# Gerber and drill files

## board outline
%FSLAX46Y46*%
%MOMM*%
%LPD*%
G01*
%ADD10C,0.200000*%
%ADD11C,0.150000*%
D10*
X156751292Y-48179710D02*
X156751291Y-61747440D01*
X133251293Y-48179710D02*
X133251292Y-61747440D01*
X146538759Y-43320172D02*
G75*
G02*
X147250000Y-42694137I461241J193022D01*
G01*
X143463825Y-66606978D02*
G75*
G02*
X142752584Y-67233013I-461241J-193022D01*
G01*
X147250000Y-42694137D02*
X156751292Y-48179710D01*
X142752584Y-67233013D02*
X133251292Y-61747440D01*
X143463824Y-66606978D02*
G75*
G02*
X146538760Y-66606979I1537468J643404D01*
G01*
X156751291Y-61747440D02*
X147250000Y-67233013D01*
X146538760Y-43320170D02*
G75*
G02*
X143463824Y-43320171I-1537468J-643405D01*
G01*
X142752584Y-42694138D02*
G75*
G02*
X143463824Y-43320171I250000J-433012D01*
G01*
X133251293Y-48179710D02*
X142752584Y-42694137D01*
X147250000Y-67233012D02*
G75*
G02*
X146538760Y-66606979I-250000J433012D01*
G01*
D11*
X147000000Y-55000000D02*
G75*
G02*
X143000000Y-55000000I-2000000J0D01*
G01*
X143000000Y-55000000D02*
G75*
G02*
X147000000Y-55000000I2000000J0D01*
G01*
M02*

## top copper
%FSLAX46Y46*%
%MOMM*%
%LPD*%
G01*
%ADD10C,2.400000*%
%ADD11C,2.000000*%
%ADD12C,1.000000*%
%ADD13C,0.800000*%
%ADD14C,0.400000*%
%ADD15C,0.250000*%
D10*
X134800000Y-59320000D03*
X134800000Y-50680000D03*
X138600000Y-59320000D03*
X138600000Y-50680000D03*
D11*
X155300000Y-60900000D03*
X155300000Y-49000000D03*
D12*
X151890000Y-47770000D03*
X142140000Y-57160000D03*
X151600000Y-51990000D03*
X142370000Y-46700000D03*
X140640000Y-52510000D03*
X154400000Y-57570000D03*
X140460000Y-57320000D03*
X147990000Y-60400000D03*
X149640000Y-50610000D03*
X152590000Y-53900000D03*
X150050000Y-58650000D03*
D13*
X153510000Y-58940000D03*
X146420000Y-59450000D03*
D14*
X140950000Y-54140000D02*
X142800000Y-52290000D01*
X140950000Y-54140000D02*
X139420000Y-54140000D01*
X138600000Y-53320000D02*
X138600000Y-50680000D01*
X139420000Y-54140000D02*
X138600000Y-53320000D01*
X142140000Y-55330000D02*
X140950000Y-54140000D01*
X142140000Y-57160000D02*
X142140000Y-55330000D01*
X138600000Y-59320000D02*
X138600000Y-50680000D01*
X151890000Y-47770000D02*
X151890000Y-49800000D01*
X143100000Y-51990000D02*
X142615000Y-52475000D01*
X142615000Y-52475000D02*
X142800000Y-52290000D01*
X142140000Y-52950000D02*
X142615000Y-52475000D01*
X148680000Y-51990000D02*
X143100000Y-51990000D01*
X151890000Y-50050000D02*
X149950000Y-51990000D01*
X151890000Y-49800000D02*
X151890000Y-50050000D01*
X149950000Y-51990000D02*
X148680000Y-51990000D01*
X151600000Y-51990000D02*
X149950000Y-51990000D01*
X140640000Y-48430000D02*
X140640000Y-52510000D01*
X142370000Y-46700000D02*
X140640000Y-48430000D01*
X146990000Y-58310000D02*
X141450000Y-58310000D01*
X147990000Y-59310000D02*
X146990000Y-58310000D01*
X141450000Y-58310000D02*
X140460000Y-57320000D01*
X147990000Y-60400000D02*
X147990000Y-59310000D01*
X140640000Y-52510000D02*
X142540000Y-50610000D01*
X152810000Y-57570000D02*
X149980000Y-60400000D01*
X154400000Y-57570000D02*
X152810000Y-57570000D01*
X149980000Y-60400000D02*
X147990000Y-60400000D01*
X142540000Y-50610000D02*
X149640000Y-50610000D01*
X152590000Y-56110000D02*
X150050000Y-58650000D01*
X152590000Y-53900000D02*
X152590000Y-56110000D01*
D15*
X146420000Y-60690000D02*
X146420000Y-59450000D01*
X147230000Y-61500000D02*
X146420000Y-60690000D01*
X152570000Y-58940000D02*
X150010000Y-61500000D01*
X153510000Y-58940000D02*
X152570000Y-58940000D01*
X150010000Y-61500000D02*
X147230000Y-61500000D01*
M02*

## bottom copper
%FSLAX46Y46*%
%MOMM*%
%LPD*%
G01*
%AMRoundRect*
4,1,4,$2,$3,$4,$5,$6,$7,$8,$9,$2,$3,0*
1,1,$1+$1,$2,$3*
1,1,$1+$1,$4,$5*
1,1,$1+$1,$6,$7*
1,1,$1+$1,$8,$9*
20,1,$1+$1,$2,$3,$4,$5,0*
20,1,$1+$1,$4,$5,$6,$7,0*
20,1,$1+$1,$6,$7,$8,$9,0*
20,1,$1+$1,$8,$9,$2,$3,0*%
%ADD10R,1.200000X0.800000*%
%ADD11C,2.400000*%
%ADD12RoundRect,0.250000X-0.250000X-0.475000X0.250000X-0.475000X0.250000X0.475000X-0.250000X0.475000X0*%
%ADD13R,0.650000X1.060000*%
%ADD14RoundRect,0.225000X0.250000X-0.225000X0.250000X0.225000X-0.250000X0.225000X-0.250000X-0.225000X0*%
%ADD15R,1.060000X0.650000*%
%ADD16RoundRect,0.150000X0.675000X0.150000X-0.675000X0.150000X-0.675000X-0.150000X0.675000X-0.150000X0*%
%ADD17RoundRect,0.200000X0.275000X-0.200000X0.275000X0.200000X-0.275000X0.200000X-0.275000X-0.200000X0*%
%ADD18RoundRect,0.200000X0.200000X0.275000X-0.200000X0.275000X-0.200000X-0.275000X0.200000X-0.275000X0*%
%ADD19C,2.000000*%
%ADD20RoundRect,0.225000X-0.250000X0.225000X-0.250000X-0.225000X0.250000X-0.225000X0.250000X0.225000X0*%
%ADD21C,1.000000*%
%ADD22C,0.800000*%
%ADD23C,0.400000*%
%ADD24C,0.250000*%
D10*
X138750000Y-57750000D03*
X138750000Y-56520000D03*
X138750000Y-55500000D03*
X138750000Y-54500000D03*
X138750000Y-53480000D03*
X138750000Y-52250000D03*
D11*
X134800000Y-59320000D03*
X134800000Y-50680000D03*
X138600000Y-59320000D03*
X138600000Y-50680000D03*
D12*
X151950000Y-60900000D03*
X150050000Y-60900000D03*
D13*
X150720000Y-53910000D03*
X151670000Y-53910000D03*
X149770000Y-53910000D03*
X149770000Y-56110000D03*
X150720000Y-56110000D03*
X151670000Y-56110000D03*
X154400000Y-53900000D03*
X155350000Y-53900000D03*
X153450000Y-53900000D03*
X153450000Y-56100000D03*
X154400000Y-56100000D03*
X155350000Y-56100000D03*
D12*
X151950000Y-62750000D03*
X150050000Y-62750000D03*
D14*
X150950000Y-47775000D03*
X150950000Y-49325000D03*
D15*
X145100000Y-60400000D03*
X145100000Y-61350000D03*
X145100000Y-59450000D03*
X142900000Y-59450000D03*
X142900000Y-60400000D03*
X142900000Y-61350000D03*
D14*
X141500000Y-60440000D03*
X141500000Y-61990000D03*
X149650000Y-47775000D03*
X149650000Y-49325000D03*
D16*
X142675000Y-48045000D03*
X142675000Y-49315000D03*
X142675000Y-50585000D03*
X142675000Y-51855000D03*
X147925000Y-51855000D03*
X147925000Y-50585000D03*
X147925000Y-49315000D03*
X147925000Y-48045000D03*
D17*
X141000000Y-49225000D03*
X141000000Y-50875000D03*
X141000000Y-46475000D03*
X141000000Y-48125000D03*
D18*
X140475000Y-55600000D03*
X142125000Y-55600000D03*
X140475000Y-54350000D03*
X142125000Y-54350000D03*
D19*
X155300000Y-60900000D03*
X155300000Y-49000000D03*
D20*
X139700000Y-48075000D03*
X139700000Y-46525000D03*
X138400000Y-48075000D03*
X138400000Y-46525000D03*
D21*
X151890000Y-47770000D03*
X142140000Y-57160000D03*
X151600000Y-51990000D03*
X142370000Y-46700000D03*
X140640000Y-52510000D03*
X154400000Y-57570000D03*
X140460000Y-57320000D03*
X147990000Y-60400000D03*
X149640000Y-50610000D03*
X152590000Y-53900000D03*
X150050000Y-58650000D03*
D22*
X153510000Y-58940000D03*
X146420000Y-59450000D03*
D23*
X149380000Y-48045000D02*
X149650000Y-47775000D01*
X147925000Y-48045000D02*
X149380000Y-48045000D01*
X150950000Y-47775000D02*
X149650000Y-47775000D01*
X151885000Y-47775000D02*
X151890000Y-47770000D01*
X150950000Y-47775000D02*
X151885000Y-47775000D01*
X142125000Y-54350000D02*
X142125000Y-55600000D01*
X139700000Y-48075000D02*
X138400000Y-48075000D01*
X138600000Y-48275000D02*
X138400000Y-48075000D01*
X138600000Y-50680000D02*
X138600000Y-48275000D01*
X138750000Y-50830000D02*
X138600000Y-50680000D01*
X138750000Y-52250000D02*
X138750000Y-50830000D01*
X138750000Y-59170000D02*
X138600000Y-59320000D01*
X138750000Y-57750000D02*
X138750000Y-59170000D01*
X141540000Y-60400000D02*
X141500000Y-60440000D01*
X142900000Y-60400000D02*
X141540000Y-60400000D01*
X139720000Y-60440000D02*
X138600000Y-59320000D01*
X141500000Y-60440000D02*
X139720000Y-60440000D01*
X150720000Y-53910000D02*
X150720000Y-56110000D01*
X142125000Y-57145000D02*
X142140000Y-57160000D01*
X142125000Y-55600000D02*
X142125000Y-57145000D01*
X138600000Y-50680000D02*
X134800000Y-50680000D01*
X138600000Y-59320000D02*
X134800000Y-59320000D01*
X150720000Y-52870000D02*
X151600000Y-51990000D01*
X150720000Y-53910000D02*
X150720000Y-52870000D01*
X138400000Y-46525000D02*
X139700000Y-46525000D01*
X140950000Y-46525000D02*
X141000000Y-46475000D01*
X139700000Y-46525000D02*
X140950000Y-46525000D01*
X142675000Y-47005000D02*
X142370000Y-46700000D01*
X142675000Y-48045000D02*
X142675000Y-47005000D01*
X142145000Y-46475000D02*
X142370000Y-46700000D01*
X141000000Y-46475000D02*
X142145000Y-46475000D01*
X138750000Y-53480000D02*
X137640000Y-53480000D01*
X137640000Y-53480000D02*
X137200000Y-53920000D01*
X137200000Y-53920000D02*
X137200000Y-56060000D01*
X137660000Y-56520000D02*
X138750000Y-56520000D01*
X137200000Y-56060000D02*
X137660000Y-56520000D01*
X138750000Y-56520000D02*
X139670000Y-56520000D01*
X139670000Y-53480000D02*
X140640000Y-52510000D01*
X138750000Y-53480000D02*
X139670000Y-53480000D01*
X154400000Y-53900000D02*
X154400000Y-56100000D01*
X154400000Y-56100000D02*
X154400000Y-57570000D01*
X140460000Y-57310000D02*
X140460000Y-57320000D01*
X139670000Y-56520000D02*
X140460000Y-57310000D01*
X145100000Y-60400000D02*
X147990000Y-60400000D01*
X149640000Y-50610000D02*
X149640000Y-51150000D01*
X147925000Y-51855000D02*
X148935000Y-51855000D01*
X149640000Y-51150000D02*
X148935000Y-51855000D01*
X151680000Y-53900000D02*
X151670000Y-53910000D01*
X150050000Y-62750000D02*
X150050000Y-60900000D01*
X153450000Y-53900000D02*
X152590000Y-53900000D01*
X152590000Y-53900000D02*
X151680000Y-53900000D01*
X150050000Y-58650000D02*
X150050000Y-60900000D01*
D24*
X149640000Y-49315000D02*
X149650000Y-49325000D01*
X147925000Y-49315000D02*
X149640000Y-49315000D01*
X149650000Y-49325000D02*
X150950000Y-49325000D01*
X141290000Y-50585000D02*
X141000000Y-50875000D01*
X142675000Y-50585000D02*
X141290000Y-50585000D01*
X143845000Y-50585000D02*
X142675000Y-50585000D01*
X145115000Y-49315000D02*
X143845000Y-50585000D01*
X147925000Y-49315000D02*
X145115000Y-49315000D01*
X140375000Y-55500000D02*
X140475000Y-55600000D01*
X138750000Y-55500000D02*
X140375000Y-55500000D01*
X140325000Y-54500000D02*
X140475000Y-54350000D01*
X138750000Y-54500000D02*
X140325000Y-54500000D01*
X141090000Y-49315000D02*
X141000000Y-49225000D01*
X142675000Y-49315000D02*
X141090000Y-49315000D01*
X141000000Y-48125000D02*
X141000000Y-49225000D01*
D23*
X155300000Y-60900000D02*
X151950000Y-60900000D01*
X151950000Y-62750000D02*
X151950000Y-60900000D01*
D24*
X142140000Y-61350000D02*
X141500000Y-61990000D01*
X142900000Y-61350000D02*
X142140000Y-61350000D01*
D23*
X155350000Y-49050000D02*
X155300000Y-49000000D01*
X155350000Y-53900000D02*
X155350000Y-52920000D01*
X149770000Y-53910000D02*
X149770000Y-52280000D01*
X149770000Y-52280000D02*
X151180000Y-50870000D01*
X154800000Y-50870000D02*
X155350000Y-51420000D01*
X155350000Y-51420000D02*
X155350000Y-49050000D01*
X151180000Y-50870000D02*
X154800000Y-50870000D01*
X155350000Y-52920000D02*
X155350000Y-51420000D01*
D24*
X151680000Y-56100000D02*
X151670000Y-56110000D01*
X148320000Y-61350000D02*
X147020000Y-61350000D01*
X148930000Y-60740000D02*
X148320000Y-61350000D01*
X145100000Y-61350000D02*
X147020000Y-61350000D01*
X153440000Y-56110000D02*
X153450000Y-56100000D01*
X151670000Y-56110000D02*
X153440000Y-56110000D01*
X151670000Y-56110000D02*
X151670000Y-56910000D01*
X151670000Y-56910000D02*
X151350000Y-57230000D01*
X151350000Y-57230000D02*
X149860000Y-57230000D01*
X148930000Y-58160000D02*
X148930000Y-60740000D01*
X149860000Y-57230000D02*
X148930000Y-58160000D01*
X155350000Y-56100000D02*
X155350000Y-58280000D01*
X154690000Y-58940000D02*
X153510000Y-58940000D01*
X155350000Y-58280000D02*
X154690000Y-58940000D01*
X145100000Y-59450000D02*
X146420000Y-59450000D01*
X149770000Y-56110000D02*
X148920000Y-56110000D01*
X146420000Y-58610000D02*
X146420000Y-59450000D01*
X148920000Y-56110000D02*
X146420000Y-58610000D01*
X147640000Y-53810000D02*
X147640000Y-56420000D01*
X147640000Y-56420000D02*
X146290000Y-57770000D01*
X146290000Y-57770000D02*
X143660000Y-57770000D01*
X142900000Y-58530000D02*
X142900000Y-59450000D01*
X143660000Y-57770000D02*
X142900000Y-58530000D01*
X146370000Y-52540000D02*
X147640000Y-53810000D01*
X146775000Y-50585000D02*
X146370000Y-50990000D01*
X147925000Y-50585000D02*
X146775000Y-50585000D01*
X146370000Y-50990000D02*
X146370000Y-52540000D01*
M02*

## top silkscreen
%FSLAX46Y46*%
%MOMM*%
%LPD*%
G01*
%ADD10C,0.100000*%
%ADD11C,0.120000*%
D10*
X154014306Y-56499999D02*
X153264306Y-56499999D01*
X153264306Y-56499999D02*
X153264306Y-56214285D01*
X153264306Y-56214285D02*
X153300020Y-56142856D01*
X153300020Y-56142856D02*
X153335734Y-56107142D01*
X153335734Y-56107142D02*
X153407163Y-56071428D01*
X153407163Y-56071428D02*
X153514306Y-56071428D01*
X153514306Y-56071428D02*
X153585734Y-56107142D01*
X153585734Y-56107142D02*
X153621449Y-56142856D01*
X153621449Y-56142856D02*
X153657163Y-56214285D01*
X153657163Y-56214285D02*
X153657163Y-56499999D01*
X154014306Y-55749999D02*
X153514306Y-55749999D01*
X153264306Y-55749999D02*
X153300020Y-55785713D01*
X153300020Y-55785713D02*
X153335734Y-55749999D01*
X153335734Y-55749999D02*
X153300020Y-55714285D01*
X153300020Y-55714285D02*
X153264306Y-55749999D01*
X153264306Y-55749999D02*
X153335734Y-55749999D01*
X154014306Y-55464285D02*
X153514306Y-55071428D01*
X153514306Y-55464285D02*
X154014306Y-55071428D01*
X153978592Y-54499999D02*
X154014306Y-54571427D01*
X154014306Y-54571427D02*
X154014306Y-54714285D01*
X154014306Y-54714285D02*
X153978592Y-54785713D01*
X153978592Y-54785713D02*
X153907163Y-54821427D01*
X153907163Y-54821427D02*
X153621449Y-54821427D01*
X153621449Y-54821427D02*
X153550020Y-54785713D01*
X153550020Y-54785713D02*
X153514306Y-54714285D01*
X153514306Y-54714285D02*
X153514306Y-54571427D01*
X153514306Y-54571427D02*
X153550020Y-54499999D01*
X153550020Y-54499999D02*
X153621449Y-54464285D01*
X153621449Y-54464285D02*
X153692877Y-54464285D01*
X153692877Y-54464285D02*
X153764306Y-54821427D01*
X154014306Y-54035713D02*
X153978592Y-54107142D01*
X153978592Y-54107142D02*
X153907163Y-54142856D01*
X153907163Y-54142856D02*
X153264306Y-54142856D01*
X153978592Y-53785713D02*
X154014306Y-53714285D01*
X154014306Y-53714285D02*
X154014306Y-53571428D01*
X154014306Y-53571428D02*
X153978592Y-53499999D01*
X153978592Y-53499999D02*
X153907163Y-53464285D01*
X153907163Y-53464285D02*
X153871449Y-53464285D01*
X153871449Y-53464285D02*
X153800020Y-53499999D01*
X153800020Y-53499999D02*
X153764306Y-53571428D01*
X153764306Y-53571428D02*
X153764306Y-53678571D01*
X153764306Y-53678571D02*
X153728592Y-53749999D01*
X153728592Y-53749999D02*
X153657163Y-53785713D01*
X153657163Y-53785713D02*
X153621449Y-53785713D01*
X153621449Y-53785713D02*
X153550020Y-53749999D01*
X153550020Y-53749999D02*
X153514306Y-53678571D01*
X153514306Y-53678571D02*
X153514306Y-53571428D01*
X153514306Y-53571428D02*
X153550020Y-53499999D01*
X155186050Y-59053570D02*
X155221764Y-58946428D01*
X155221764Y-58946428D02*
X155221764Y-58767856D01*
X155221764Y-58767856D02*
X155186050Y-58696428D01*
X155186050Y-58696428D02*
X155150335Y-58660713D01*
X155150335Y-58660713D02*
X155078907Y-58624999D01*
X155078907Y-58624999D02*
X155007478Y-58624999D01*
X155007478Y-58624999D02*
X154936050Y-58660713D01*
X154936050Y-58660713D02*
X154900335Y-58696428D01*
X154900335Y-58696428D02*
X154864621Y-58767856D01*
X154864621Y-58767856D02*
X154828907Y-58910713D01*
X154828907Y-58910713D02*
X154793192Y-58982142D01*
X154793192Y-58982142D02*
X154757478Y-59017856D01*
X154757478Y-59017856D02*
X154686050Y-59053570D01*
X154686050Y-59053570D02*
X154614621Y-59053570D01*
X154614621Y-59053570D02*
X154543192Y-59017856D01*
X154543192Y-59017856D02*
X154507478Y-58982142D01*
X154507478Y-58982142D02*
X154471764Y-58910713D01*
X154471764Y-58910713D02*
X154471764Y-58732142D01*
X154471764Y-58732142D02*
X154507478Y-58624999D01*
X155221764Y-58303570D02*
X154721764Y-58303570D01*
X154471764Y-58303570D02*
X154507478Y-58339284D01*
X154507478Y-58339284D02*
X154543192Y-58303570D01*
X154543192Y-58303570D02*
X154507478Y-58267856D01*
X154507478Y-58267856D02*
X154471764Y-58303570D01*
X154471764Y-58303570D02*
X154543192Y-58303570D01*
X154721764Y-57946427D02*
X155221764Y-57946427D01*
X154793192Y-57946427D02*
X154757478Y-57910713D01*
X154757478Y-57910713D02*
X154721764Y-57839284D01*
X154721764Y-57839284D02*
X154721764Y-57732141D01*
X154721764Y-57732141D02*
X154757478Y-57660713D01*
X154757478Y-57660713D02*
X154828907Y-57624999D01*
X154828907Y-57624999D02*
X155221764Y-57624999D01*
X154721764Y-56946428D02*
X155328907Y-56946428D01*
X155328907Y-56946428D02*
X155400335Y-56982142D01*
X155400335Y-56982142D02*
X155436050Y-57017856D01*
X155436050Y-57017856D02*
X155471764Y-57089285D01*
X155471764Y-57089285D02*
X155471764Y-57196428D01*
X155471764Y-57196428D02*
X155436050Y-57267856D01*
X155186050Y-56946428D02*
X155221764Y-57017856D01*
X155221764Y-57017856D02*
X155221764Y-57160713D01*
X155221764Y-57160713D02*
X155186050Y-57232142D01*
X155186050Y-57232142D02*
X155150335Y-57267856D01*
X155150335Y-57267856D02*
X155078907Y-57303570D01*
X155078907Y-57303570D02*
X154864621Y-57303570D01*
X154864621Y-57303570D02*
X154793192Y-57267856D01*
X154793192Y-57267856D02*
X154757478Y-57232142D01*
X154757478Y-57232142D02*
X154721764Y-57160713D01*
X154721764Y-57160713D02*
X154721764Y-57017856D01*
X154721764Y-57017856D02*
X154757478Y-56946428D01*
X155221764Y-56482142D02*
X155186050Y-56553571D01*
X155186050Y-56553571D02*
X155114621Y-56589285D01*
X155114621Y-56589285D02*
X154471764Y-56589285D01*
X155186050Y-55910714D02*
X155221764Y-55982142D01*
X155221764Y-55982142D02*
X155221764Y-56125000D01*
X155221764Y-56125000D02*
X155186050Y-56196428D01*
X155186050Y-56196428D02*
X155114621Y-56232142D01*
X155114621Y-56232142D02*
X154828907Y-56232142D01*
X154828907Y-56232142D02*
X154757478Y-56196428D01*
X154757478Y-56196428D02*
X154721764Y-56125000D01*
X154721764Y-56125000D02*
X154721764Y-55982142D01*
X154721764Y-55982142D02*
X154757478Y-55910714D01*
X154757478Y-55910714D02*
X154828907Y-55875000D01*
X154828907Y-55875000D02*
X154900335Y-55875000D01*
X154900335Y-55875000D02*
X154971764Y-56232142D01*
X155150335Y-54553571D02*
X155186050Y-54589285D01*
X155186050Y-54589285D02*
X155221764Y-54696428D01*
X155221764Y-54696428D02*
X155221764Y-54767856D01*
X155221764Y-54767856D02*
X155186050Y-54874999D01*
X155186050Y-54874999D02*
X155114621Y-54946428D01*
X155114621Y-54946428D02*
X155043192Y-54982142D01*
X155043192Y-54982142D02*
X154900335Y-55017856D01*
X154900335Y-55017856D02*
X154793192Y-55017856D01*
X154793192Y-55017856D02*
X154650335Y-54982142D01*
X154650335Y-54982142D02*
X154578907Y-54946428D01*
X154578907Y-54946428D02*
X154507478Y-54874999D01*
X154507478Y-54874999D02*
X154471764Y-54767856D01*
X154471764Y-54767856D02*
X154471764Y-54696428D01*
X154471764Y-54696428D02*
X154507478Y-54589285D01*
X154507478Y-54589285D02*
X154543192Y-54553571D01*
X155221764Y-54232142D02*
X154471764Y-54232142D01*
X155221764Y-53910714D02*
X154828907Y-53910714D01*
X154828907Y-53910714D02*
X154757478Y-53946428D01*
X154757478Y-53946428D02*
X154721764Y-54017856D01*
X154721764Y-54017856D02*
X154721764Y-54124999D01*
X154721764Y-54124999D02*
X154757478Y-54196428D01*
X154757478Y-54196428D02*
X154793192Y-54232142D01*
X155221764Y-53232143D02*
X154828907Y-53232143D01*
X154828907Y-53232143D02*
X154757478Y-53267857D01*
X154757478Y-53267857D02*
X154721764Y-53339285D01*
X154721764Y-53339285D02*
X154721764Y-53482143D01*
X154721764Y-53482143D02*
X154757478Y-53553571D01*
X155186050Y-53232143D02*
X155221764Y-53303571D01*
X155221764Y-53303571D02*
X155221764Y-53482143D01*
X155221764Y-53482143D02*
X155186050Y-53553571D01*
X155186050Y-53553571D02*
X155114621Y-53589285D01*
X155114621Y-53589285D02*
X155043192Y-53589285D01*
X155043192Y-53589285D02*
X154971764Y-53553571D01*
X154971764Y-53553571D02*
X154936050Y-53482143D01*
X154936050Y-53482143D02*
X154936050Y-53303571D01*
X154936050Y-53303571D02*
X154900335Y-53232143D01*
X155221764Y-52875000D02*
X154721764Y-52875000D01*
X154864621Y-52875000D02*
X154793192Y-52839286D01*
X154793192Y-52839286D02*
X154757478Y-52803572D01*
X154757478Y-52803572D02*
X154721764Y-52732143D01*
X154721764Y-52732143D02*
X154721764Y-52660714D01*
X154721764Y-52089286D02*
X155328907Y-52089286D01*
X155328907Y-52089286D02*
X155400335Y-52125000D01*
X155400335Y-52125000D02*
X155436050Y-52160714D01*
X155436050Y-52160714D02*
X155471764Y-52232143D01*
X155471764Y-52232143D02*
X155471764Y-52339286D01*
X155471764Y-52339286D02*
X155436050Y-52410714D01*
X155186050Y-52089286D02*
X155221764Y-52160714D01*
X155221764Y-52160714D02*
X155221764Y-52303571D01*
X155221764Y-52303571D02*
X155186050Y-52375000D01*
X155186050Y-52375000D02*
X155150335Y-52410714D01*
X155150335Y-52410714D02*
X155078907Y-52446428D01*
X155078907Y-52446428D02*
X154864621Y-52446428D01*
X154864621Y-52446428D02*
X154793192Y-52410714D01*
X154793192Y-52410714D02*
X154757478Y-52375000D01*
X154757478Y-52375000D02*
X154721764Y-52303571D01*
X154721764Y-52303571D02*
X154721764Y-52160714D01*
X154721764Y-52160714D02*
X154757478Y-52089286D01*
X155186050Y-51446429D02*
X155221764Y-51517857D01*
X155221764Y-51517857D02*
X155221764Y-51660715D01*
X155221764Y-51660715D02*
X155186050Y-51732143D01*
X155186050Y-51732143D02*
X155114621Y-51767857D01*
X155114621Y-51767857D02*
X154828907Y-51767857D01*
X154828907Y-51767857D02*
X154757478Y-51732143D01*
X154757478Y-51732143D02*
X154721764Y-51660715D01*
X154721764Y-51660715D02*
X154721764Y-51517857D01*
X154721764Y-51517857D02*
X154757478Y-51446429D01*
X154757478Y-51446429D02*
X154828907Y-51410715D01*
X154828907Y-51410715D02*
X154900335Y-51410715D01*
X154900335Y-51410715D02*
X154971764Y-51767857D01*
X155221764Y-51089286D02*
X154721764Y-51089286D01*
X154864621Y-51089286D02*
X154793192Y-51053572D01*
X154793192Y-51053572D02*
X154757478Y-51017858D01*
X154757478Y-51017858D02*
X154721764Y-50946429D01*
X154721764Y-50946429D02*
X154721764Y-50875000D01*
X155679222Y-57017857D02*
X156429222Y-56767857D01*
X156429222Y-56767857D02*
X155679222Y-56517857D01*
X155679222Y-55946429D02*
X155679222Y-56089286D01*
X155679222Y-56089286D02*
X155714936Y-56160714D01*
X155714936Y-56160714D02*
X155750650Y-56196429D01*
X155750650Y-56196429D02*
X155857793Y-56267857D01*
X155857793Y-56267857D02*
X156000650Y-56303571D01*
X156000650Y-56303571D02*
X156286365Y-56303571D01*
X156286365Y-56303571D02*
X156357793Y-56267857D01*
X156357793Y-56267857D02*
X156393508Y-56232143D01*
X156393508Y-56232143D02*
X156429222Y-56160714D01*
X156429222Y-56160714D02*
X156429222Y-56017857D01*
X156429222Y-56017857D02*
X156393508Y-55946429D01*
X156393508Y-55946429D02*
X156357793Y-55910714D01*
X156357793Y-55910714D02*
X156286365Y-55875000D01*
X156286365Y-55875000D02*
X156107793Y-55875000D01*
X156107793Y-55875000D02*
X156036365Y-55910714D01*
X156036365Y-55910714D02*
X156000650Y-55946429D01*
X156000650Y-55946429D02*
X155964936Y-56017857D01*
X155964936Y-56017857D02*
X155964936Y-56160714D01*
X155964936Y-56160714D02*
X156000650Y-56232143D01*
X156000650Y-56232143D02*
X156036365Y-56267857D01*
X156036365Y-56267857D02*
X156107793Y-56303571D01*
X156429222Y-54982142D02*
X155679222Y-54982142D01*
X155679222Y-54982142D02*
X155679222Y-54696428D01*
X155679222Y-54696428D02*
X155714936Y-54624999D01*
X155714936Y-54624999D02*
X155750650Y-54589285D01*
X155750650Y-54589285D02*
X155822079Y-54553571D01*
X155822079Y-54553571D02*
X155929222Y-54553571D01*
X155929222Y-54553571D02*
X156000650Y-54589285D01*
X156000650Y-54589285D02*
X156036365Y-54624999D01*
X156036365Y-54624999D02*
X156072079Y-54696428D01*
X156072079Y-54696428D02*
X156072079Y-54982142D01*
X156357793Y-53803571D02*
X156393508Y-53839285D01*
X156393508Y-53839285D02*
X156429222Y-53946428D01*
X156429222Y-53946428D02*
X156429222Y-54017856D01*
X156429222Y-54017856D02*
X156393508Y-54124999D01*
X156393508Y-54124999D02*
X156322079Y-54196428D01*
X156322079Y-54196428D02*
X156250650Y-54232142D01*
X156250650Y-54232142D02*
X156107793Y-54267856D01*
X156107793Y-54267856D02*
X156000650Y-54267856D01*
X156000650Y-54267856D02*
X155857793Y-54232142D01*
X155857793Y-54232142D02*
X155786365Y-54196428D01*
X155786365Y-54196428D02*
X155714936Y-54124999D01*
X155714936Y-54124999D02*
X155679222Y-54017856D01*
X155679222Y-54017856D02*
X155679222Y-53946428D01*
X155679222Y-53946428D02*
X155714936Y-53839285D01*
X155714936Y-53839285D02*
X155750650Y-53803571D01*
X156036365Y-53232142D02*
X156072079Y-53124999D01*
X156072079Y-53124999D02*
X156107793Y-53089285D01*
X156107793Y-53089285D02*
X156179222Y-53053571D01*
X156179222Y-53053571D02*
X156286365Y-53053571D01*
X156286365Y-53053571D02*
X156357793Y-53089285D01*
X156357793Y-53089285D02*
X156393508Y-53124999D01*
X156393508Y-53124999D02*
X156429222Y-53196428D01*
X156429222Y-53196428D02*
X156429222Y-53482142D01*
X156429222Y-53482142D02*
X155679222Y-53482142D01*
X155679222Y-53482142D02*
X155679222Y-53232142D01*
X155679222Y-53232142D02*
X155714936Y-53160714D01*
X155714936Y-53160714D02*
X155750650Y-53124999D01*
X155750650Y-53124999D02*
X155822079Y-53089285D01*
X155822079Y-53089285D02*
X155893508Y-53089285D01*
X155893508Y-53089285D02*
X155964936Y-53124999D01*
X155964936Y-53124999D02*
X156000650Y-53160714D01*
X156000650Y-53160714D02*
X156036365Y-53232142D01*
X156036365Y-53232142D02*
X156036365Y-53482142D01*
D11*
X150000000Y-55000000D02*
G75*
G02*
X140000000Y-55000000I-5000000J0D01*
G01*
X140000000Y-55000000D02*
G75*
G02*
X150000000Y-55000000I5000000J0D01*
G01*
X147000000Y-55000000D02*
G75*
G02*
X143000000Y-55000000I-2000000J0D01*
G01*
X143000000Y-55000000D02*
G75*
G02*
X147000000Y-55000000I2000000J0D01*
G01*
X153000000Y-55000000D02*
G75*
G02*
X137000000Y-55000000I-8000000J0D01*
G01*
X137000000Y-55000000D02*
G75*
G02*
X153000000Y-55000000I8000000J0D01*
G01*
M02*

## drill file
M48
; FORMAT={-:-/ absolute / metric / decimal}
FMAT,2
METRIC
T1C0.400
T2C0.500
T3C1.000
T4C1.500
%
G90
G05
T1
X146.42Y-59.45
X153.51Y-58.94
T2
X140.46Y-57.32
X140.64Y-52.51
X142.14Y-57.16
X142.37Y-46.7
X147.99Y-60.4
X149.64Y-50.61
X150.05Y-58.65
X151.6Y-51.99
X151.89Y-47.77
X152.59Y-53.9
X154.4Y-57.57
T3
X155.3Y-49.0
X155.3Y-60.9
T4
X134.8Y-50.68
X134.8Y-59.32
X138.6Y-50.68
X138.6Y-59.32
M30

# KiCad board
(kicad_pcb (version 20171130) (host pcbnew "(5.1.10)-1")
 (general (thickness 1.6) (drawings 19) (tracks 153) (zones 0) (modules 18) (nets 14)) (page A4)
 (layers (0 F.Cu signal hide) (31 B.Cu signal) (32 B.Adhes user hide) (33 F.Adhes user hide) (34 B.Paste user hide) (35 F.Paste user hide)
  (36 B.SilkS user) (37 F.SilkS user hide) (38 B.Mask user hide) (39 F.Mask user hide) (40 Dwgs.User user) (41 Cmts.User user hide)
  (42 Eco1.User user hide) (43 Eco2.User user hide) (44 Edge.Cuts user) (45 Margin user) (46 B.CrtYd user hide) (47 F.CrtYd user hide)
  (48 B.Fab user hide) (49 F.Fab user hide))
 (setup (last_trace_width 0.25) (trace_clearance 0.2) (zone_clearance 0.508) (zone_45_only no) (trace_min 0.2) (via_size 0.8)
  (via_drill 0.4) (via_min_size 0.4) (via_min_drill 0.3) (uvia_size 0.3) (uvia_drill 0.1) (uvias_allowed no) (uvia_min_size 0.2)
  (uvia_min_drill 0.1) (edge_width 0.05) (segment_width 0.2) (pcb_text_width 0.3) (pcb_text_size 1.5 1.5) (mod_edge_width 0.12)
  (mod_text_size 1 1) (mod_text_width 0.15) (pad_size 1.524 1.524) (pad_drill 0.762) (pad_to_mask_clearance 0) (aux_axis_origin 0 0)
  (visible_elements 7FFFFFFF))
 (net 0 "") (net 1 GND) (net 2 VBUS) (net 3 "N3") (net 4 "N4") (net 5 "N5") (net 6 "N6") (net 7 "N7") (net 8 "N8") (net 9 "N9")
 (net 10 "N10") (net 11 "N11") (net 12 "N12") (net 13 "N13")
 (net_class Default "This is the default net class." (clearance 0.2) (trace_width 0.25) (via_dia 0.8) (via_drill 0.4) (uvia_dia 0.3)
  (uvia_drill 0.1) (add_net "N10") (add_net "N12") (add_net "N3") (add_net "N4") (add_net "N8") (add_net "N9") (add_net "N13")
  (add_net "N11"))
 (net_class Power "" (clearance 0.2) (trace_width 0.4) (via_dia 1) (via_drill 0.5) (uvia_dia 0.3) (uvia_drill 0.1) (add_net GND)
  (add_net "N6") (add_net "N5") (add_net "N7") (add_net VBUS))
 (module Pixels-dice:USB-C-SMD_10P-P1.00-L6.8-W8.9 (layer B.Cu) (at 136.7 55)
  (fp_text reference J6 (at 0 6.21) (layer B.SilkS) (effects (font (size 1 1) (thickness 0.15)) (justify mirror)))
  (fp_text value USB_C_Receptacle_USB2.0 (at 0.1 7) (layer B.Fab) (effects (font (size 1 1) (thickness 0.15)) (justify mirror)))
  (pad B12 smd rect (at 2.05 2.75 90) (size 0.8 1.2) (layers B.Cu B.Paste B.Mask) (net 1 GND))
  (pad B9 smd rect (at 2.05 1.52 90) (size 0.8 1.2) (layers B.Cu B.Paste B.Mask) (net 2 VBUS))
  (pad A5 smd rect (at 2.05 0.5 90) (size 0.8 1.2) (layers B.Cu B.Paste B.Mask) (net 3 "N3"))
  (pad B5 smd rect (at 2.05 -0.5 90) (size 0.8 1.2) (layers B.Cu B.Paste B.Mask) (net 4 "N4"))
  (pad A9 smd rect (at 2.05 -1.52 90) (size 0.8 1.2) (layers B.Cu B.Paste B.Mask) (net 2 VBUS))
  (pad A12 smd rect (at 2.05 -2.75 90) (size 0.8 1.2) (layers B.Cu B.Paste B.Mask) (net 1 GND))
  (pad S1 thru_hole circle (at -1.9 4.32 90) (size 2.4 2.4) (drill 1.5) (layers *.Cu *.Mask) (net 1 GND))
  (pad S1 thru_hole circle (at -1.9 -4.32 90) (size 2.4 2.4) (drill 1.5) (layers *.Cu *.Mask) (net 1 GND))
  (pad S1 thru_hole circle (at 1.9 4.32 90) (size 2.4 2.4) (drill 1.5) (layers *.Cu *.Mask) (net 1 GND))
  (pad S1 thru_hole circle (at 1.9 -4.32 90) (size 2.4 2.4) (drill 1.5) (layers *.Cu *.Mask) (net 1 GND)))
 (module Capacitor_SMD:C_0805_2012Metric (layer B.Cu) (at 151 60.9)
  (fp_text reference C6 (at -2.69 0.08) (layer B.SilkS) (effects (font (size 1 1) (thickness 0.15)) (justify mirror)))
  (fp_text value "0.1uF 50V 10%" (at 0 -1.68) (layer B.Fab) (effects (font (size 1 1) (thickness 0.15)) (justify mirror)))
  (pad 2 smd roundrect (at 0.95 0) (size 1 1.45) (layers B.Cu B.Paste B.Mask) (roundrect_rratio 0.25) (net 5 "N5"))
  (pad 1 smd roundrect (at -0.95 0) (size 1 1.45) (layers B.Cu B.Paste B.Mask) (roundrect_rratio 0.25) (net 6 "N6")))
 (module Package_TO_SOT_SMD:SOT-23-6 (layer B.Cu) (at 150.72 55.01 90)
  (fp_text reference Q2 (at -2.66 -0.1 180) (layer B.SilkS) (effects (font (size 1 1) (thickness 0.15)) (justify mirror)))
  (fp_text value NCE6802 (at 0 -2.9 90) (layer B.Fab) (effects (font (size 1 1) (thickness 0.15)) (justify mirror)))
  (pad 5 smd rect (at 1.1 0 90) (size 1.06 0.65) (layers B.Cu B.Paste B.Mask) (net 1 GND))
  (pad 6 smd rect (at 1.1 0.95 90) (size 1.06 0.65) (layers B.Cu B.Paste B.Mask) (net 6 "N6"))
  (pad 4 smd rect (at 1.1 -0.95 90) (size 1.06 0.65) (layers B.Cu B.Paste B.Mask) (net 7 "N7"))
  (pad 3 smd rect (at -1.1 -0.95 90) (size 1.06 0.65) (layers B.Cu B.Paste B.Mask) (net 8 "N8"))
  (pad 2 smd rect (at -1.1 0 90) (size 1.06 0.65) (layers B.Cu B.Paste B.Mask) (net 1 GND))
  (pad 1 smd rect (at -1.1 0.95 90) (size 1.06 0.65) (layers B.Cu B.Paste B.Mask) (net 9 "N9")))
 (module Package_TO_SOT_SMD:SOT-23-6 (layer B.Cu) (at 154.4 55 90)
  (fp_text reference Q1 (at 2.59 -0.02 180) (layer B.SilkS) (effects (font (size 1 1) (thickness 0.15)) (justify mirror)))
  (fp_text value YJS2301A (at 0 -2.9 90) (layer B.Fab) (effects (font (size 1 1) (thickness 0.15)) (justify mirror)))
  (pad 5 smd rect (at 1.1 0 90) (size 1.06 0.65) (layers B.Cu B.Paste B.Mask) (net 2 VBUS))
  (pad 6 smd rect (at 1.1 0.95 90) (size 1.06 0.65) (layers B.Cu B.Paste B.Mask) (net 7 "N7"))
  (pad 4 smd rect (at 1.1 -0.95 90) (size 1.06 0.65) (layers B.Cu B.Paste B.Mask) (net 6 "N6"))
  (pad 3 smd rect (at -1.1 -0.95 90) (size 1.06 0.65) (layers B.Cu B.Paste B.Mask) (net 9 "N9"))
  (pad 2 smd rect (at -1.1 0 90) (size 1.06 0.65) (layers B.Cu B.Paste B.Mask) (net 2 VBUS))
  (pad 1 smd rect (at -1.1 0.95 90) (size 1.06 0.65) (layers B.Cu B.Paste B.Mask) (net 8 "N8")))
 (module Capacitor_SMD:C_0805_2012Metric (layer B.Cu) (at 151 62.75)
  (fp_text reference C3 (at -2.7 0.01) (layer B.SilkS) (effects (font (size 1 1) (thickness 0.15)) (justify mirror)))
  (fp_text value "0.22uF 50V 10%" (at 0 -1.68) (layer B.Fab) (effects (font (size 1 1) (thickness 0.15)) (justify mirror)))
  (pad 2 smd roundrect (at 0.95 0) (size 1 1.45) (layers B.Cu B.Paste B.Mask) (roundrect_rratio 0.25) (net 5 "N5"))
  (pad 1 smd roundrect (at -0.95 0) (size 1 1.45) (layers B.Cu B.Paste B.Mask) (roundrect_rratio 0.25) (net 6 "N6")))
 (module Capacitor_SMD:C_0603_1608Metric (layer B.Cu) (at 150.95 48.55 90)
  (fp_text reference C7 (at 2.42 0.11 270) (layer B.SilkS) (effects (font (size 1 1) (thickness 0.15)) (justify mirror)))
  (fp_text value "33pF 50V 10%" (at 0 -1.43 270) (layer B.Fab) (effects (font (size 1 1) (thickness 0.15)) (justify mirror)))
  (pad 2 smd roundrect (at 0.775 0 90) (size 0.9 0.95) (layers B.Cu B.Paste B.Mask) (roundrect_rratio 0.25) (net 1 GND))
  (pad 1 smd roundrect (at -0.775 0 90) (size 0.9 0.95) (layers B.Cu B.Paste B.Mask) (roundrect_rratio 0.25) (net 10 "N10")))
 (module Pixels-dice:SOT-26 (layer B.Cu) (at 144 60.4 180)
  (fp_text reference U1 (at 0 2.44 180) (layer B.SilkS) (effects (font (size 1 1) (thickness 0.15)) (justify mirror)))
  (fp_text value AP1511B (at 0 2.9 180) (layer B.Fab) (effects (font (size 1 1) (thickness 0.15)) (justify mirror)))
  (pad 5 smd rect (at -1.1 0) (size 1.06 0.65) (layers B.Cu B.Paste B.Mask) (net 2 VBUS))
  (pad 6 smd rect (at -1.1 -0.95) (size 1.06 0.65) (layers B.Cu B.Paste B.Mask) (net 9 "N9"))
  (pad 4 smd rect (at -1.1 0.95) (size 1.06 0.65) (layers B.Cu B.Paste B.Mask) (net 8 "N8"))
  (pad 3 smd rect (at 1.1 0.95) (size 1.06 0.65) (layers B.Cu B.Paste B.Mask) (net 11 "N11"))
  (pad 2 smd rect (at 1.1 0) (size 1.06 0.65) (layers B.Cu B.Paste B.Mask) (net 1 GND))
  (pad 1 smd rect (at 1.1 -0.95) (size 1.06 0.65) (layers B.Cu B.Paste B.Mask) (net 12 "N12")))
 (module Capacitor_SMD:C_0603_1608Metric (layer B.Cu) (at 141.5 61.215 90)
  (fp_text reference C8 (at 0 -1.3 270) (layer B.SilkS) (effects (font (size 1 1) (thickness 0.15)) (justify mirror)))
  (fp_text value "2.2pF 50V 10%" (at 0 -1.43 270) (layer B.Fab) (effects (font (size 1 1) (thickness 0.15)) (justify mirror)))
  (pad 2 smd roundrect (at 0.775 0 90) (size 0.9 0.95) (layers B.Cu B.Paste B.Mask) (roundrect_rratio 0.25) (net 1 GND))
  (pad 1 smd roundrect (at -0.775 0 90) (size 0.9 0.95) (layers B.Cu B.Paste B.Mask) (roundrect_rratio 0.25) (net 12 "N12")))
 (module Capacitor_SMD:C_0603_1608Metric (layer B.Cu) (at 149.65 48.55 90)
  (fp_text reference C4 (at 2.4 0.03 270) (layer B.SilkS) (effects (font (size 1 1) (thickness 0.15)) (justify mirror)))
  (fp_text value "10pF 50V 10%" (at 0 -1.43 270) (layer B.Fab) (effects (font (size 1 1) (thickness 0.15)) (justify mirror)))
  (pad 2 smd roundrect (at 0.775 0 90) (size 0.9 0.95) (layers B.Cu B.Paste B.Mask) (roundrect_rratio 0.25) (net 1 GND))
  (pad 1 smd roundrect (at -0.775 0 90) (size 0.9 0.95) (layers B.Cu B.Paste B.Mask) (roundrect_rratio 0.25) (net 10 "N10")))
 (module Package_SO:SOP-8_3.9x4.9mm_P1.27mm (layer B.Cu) (at 145.3 49.95 180)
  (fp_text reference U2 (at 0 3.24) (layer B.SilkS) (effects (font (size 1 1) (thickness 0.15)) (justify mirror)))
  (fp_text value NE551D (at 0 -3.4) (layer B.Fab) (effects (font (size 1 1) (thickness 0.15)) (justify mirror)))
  (pad 8 smd roundrect (at 2.625 1.905 180) (size 1.65 0.6) (layers B.Cu B.Paste B.Mask) (roundrect_rratio 0.25) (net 2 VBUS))
  (pad 7 smd roundrect (at 2.625 0.635 180) (size 1.65 0.6) (layers B.Cu B.Paste B.Mask) (roundrect_rratio 0.25) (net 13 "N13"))
  (pad 6 smd roundrect (at 2.625 -0.635 180) (size 1.65 0.6) (layers B.Cu B.Paste B.Mask) (roundrect_rratio 0.25) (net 10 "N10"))
  (pad 5 smd roundrect (at 2.625 -1.905 180) (size 1.65 0.6) (layers B.Cu B.Paste B.Mask) (roundrect_rratio 0.25))
  (pad 4 smd roundrect (at -2.625 -1.905 180) (size 1.65 0.6) (layers B.Cu B.Paste B.Mask) (roundrect_rratio 0.25) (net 2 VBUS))
  (pad 3 smd roundrect (at -2.625 -0.635 180) (size 1.65 0.6) (layers B.Cu B.Paste B.Mask) (roundrect_rratio 0.25) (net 11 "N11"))
  (pad 2 smd roundrect (at -2.625 0.635 180) (size 1.65 0.6) (layers B.Cu B.Paste B.Mask) (roundrect_rratio 0.25) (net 10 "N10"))
  (pad 1 smd roundrect (at -2.625 1.905 180) (size 1.65 0.6) (layers B.Cu B.Paste B.Mask) (roundrect_rratio 0.25) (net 1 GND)))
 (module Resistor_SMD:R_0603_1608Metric (layer B.Cu) (at 141 50.05 90)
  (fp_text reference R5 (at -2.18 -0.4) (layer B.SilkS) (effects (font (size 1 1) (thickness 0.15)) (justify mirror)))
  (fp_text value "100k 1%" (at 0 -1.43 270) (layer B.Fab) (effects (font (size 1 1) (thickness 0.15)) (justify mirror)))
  (pad 2 smd roundrect (at 0.825 0 90) (size 0.8 0.95) (layers B.Cu B.Paste B.Mask) (roundrect_rratio 0.25) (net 13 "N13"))
  (pad 1 smd roundrect (at -0.825 0 90) (size 0.8 0.95) (layers B.Cu B.Paste B.Mask) (roundrect_rratio 0.25) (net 10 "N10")))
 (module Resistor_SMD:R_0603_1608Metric (layer B.Cu) (at 141 47.3 90)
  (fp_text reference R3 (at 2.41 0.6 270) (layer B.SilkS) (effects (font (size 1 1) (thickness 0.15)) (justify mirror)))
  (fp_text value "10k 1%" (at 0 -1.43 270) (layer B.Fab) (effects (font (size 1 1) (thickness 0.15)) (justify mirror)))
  (pad 2 smd roundrect (at 0.825 0 90) (size 0.8 0.95) (layers B.Cu B.Paste B.Mask) (roundrect_rratio 0.25) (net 2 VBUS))
  (pad 1 smd roundrect (at -0.825 0 90) (size 0.8 0.95) (layers B.Cu B.Paste B.Mask) (roundrect_rratio 0.25) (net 13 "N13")))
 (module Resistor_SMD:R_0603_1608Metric (layer B.Cu) (at 141.3 55.6 180)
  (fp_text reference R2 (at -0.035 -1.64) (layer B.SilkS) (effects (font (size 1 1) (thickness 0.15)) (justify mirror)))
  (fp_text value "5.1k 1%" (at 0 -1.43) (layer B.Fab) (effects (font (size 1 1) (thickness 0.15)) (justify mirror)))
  (pad 2 smd roundrect (at 0.825 0 180) (size 0.8 0.95) (layers B.Cu B.Paste B.Mask) (roundrect_rratio 0.25) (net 3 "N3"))
  (pad 1 smd roundrect (at -0.825 0 180) (size 0.8 0.95) (layers B.Cu B.Paste B.Mask) (roundrect_rratio 0.25) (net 1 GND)))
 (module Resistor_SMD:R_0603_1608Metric (layer B.Cu) (at 141.3 54.35 180)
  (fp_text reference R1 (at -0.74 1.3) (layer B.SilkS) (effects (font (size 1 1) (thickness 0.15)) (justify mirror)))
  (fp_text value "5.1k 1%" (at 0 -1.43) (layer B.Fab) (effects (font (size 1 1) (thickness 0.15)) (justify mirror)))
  (pad 2 smd roundrect (at 0.825 0 180) (size 0.8 0.95) (layers B.Cu B.Paste B.Mask) (roundrect_rratio 0.25) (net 4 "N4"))
  (pad 1 smd roundrect (at -0.825 0 180) (size 0.8 0.95) (layers B.Cu B.Paste B.Mask) (roundrect_rratio 0.25) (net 1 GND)))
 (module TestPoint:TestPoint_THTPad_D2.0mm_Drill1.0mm (layer B.Cu) (at 155.3 60.9)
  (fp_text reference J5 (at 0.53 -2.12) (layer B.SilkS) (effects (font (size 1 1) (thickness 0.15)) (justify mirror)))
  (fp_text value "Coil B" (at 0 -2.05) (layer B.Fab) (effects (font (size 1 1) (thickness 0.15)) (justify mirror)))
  (pad 1 thru_hole circle (at 0 0) (size 2 2) (drill 1) (layers *.Cu *.Mask) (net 5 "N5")))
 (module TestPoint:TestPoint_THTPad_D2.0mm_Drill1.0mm (layer B.Cu) (at 155.3 49)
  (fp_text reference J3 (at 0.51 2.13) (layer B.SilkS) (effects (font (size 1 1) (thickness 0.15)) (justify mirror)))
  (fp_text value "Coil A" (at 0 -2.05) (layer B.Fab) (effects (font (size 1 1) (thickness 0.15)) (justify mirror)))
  (pad 1 thru_hole circle (at 0 0) (size 2 2) (drill 1) (layers *.Cu *.Mask) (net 7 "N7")))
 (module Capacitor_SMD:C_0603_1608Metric (layer B.Cu) (at 139.7 47.3 270)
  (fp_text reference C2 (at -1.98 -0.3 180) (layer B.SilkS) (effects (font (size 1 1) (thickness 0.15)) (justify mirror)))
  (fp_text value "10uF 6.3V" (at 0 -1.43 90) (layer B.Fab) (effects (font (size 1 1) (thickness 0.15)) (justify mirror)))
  (pad 2 smd roundrect (at 0.775 0 270) (size 0.9 0.95) (layers B.Cu B.Paste B.Mask) (roundrect_rratio 0.25) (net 1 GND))
  (pad 1 smd roundrect (at -0.775 0 270) (size 0.9 0.95) (layers B.Cu B.Paste B.Mask) (roundrect_rratio 0.25) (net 2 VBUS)))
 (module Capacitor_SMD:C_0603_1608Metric (layer B.Cu) (at 138.4 47.3 270)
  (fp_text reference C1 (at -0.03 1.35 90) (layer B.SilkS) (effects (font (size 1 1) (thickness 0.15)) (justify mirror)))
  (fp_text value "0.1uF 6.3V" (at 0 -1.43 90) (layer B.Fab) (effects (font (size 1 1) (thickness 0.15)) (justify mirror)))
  (pad 2 smd roundrect (at 0.775 0 270) (size 0.9 0.95) (layers B.Cu B.Paste B.Mask) (roundrect_rratio 0.25) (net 1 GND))
  (pad 1 smd roundrect (at -0.775 0 270) (size 0.9 0.95) (layers B.Cu B.Paste B.Mask) (roundrect_rratio 0.25) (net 2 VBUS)))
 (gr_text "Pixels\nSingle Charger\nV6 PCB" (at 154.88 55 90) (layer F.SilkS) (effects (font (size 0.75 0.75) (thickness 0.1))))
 (gr_line (start 156.751292 48.17971) (end 156.751291 61.74744) (layer Edge.Cuts) (width 0.2))
 (gr_line (start 133.251293 48.17971) (end 133.251292 61.74744) (layer Edge.Cuts) (width 0.2))
 (gr_circle (center 145 55) (end 150 55) (layer F.SilkS) (width 0.12))
 (gr_circle (center 145 55) (end 147 55) (layer F.SilkS) (width 0.12))
 (gr_circle (center 145 55) (end 153 55) (layer F.SilkS) (width 0.12))
 (gr_arc (start 147 43.12715) (end 147.25 42.694137) (angle -142.7084941) (layer Edge.Cuts) (width 0.2))
 (gr_arc (start 143.002584 66.8) (end 142.752584 67.233013) (angle -142.7084941) (layer Edge.Cuts) (width 0.2))
 (gr_line (start 147.25 42.694137) (end 156.751292 48.17971) (layer Edge.Cuts) (width 0.2))
 (gr_line (start 142.752584 67.233013) (end 133.251292 61.74744) (layer Edge.Cuts) (width 0.2))
 (gr_arc (start 145.001292 65.963574) (end 146.53876 66.606979) (angle -225.4169678) (layer Edge.Cuts) (width 0.2))
 (gr_line (start 156.751291 61.74744) (end 147.25 67.233013) (layer Edge.Cuts) (width 0.2))
 (gr_arc (start 145.001292 43.963575) (end 143.463824 43.320171) (angle -225.4169678) (layer Edge.Cuts) (width 0.2))
 (gr_arc (start 143.002584 43.12715) (end 143.463824 43.320171) (angle -142.7084738) (layer Edge.Cuts) (width 0.2))
 (gr_line (start 133.251293 48.17971) (end 142.752584 42.694137) (layer Edge.Cuts) (width 0.2))
 (gr_arc (start 147 66.8) (end 146.53876 66.606979) (angle -142.7084738) (layer Edge.Cuts) (width 0.2))
 (gr_circle (center 145 55) (end 147 55) (layer Edge.Cuts) (width 0.15))
 (segment (start 149.38 48.045) (end 149.65 47.775) (width 0.4) (layer B.Cu) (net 1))
 (segment (start 147.925 48.045) (end 149.38 48.045) (width 0.4) (layer B.Cu) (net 1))
 (segment (start 150.95 47.775) (end 149.65 47.775) (width 0.4) (layer B.Cu) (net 1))
 (via (at 151.89 47.77) (size 1) (drill 0.5) (layers F.Cu B.Cu) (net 1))
 (segment (start 151.885 47.775) (end 151.89 47.77) (width 0.4) (layer B.Cu) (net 1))
 (segment (start 150.95 47.775) (end 151.885 47.775) (width 0.4) (layer B.Cu) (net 1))
 (segment (start 142.125 54.35) (end 142.125 55.6) (width 0.4) (layer B.Cu) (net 1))
 (via (at 142.14 57.16) (size 1) (drill 0.5) (layers F.Cu B.Cu) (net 1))
 (segment (start 139.7 48.075) (end 138.4 48.075) (width 0.4) (layer B.Cu) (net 1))
 (segment (start 138.6 48.275) (end 138.4 48.075) (width 0.4) (layer B.Cu) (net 1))
 (segment (start 138.6 50.68) (end 138.6 48.275) (width 0.4) (layer B.Cu) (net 1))
 (segment (start 138.75 50.83) (end 138.6 50.68) (width 0.4) (layer B.Cu) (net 1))
 (segment (start 138.75 52.25) (end 138.75 50.83) (width 0.4) (layer B.Cu) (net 1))
 (segment (start 138.75 59.17) (end 138.6 59.32) (width 0.4) (layer B.Cu) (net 1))
 (segment (start 138.75 57.75) (end 138.75 59.17) (width 0.4) (layer B.Cu) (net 1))
 (segment (start 141.54 60.4) (end 141.5 60.44) (width 0.4) (layer B.Cu) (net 1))
 (segment (start 142.9 60.4) (end 141.54 60.4) (width 0.4) (layer B.Cu) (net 1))
 (segment (start 139.72 60.44) (end 138.6 59.32) (width 0.4) (layer B.Cu) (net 1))
 (segment (start 141.5 60.44) (end 139.72 60.44) (width 0.4) (layer B.Cu) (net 1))
 (segment (start 150.72 53.91) (end 150.72 56.11) (width 0.4) (layer B.Cu) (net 1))
 (segment (start 140.95 54.14) (end 142.8 52.29) (width 0.4) (layer F.Cu) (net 1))
 (segment (start 140.95 54.14) (end 139.42 54.14) (width 0.4) (layer F.Cu) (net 1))
 (segment (start 138.6 53.32) (end 138.6 50.68) (width 0.4) (layer F.Cu) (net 1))
 (segment (start 139.42 54.14) (end 138.6 53.32) (width 0.4) (layer F.Cu) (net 1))
 (segment (start 142.125 57.145) (end 142.14 57.16) (width 0.4) (layer B.Cu) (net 1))
 (segment (start 142.125 55.6) (end 142.125 57.145) (width 0.4) (layer B.Cu) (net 1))
 (segment (start 138.6 50.68) (end 134.8 50.68) (width 0.4) (layer B.Cu) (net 1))
 (segment (start 138.6 59.32) (end 134.8 59.32) (width 0.4) (layer B.Cu) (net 1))
 (segment (start 142.14 55.33) (end 140.95 54.14) (width 0.4) (layer F.Cu) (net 1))
 (segment (start 142.14 57.16) (end 142.14 55.33) (width 0.4) (layer F.Cu) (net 1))
 (segment (start 138.6 59.32) (end 138.6 50.68) (width 0.4) (layer F.Cu) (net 1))
 (segment (start 151.89 47.77) (end 151.89 49.8) (width 0.4) (layer F.Cu) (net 1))
 (via (at 151.6 51.99) (size 1) (drill 0.5) (layers F.Cu B.Cu) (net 1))
 (segment (start 150.72 52.87) (end 151.6 51.99) (width 0.4) (layer B.Cu) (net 1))
 (segment (start 150.72 53.91) (end 150.72 52.87) (width 0.4) (layer B.Cu) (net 1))
 (segment (start 143.1 51.99) (end 142.615 52.475) (width 0.4) (layer F.Cu) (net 1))
 (segment (start 142.615 52.475) (end 142.8 52.29) (width 0.4) (layer F.Cu) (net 1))
 (segment (start 142.14 52.95) (end 142.615 52.475) (width 0.4) (layer F.Cu) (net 1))
 (segment (start 148.68 51.99) (end 143.1 51.99) (width 0.4) (layer F.Cu) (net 1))
 (segment (start 151.89 50.05) (end 149.95 51.99) (width 0.4) (layer F.Cu) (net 1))
 (segment (start 151.89 49.8) (end 151.89 50.05) (width 0.4) (layer F.Cu) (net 1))
 (segment (start 149.95 51.99) (end 148.68 51.99) (width 0.4) (layer F.Cu) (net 1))
 (segment (start 151.6 51.99) (end 149.95 51.99) (width 0.4) (layer F.Cu) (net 1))
 (segment (start 138.4 46.525) (end 139.7 46.525) (width 0.4) (layer B.Cu) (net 2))
 (segment (start 140.95 46.525) (end 141 46.475) (width 0.4) (layer B.Cu) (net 2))
 (segment (start 139.7 46.525) (end 140.95 46.525) (width 0.4) (layer B.Cu) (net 2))
 (segment (start 142.675 47.005) (end 142.37 46.7) (width 0.4) (layer B.Cu) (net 2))
 (via (at 142.37 46.7) (size 1) (drill 0.5) (layers F.Cu B.Cu) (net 2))
 (segment (start 142.675 48.045) (end 142.675 47.005) (width 0.4) (layer B.Cu) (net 2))
 (segment (start 142.145 46.475) (end 142.37 46.7) (width 0.4) (layer B.Cu) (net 2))
 (segment (start 141 46.475) (end 142.145 46.475) (width 0.4) (layer B.Cu) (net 2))
 (segment (start 138.75 53.48) (end 137.64 53.48) (width 0.4) (layer B.Cu) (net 2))
 (segment (start 137.64 53.48) (end 137.2 53.92) (width 0.4) (layer B.Cu) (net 2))
 (segment (start 137.2 53.92) (end 137.2 56.06) (width 0.4) (layer B.Cu) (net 2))
 (segment (start 137.66 56.52) (end 138.75 56.52) (width 0.4) (layer B.Cu) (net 2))
 (segment (start 137.2 56.06) (end 137.66 56.52) (width 0.4) (layer B.Cu) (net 2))
 (segment (start 138.75 56.52) (end 139.67 56.52) (width 0.4) (layer B.Cu) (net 2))
 (via (at 140.64 52.51) (size 1) (drill 0.5) (layers F.Cu B.Cu) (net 2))
 (segment (start 139.67 53.48) (end 140.64 52.51) (width 0.4) (layer B.Cu) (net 2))
 (segment (start 138.75 53.48) (end 139.67 53.48) (width 0.4) (layer B.Cu) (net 2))
 (segment (start 154.4 53.9) (end 154.4 56.1) (width 0.4) (layer B.Cu) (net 2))
 (via (at 154.4 57.57) (size 1) (drill 0.5) (layers F.Cu B.Cu) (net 2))
 (segment (start 154.4 56.1) (end 154.4 57.57) (width 0.4) (layer B.Cu) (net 2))
 (segment (start 140.64 48.43) (end 140.64 52.51) (width 0.4) (layer F.Cu) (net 2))
 (segment (start 142.37 46.7) (end 140.64 48.43) (width 0.4) (layer F.Cu) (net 2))
 (segment (start 140.46 57.31) (end 140.46 57.32) (width 0.4) (layer B.Cu) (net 2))
 (via (at 140.46 57.32) (size 1) (drill 0.5) (layers F.Cu B.Cu) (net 2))
 (segment (start 139.67 56.52) (end 140.46 57.31) (width 0.4) (layer B.Cu) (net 2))
 (segment (start 145.1 60.4) (end 147.99 60.4) (width 0.4) (layer B.Cu) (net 2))
 (via (at 147.99 60.4) (size 1) (drill 0.5) (layers F.Cu B.Cu) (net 2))
 (segment (start 146.99 58.31) (end 141.45 58.31) (width 0.4) (layer F.Cu) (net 2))
 (segment (start 147.99 59.31) (end 146.99 58.31) (width 0.4) (layer F.Cu) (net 2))
 (segment (start 141.45 58.31) (end 140.46 57.32) (width 0.4) (layer F.Cu) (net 2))
 (segment (start 147.99 60.4) (end 147.99 59.31) (width 0.4) (layer F.Cu) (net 2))
 (segment (start 140.64 52.51) (end 142.54 50.61) (width 0.4) (layer F.Cu) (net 2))
 (segment (start 152.81 57.57) (end 149.98 60.4) (width 0.4) (layer F.Cu) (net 2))
 (segment (start 154.4 57.57) (end 152.81 57.57) (width 0.4) (layer F.Cu) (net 2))
 (segment (start 149.98 60.4) (end 147.99 60.4) (width 0.4) (layer F.Cu) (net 2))
 (via (at 149.64 50.61) (size 1) (drill 0.5) (layers F.Cu B.Cu) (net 2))
 (segment (start 149.64 50.61) (end 149.64 51.15) (width 0.4) (layer B.Cu) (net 2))
 (segment (start 147.925 51.855) (end 148.935 51.855) (width 0.4) (layer B.Cu) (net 2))
 (segment (start 149.64 51.15) (end 148.935 51.855) (width 0.4) (layer B.Cu) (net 2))
 (segment (start 142.54 50.61) (end 149.64 50.61) (width 0.4) (layer F.Cu) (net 2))
 (segment (start 151.68 53.9) (end 151.67 53.91) (width 0.4) (layer B.Cu) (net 6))
 (segment (start 150.05 62.75) (end 150.05 60.9) (width 0.4) (layer B.Cu) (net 6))
 (segment (start 153.45 53.9) (end 152.59 53.9) (width 0.4) (layer B.Cu) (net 6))
 (segment (start 152.59 53.9) (end 151.68 53.9) (width 0.4) (layer B.Cu) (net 6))
 (via (at 152.59 53.9) (size 1) (drill 0.5) (layers F.Cu B.Cu) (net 6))
 (via (at 150.05 58.65) (size 1) (drill 0.5) (layers F.Cu B.Cu) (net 6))
 (segment (start 150.05 58.65) (end 150.05 60.9) (width 0.4) (layer B.Cu) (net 6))
 (segment (start 152.59 56.11) (end 150.05 58.65) (width 0.4) (layer F.Cu) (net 6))
 (segment (start 152.59 53.9) (end 152.59 56.11) (width 0.4) (layer F.Cu) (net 6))
 (segment (start 149.64 49.315) (end 149.65 49.325) (width 0.25) (layer B.Cu) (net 10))
 (segment (start 147.925 49.315) (end 149.64 49.315) (width 0.25) (layer B.Cu) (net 10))
 (segment (start 149.65 49.325) (end 150.95 49.325) (width 0.25) (layer B.Cu) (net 10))
 (segment (start 141.29 50.585) (end 141 50.875) (width 0.25) (layer B.Cu) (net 10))
 (segment (start 142.675 50.585) (end 141.29 50.585) (width 0.25) (layer B.Cu) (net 10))
 (segment (start 143.845 50.585) (end 142.675 50.585) (width 0.25) (layer B.Cu) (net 10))
 (segment (start 145.115 49.315) (end 143.845 50.585) (width 0.25) (layer B.Cu) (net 10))
 (segment (start 147.925 49.315) (end 145.115 49.315) (width 0.25) (layer B.Cu) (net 10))
 (segment (start 140.375 55.5) (end 140.475 55.6) (width 0.25) (layer B.Cu) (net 3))
 (segment (start 138.75 55.5) (end 140.375 55.5) (width 0.25) (layer B.Cu) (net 3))
 (segment (start 140.325 54.5) (end 140.475 54.35) (width 0.25) (layer B.Cu) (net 4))
 (segment (start 138.75 54.5) (end 140.325 54.5) (width 0.25) (layer B.Cu) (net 4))
 (segment (start 141.09 49.315) (end 141 49.225) (width 0.25) (layer B.Cu) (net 13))
 (segment (start 142.675 49.315) (end 141.09 49.315) (width 0.25) (layer B.Cu) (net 13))
 (segment (start 141 48.125) (end 141 49.225) (width 0.25) (layer B.Cu) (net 13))
 (segment (start 155.3 60.9) (end 151.95 60.9) (width 0.4) (layer B.Cu) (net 5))
 (segment (start 151.95 62.75) (end 151.95 60.9) (width 0.4) (layer B.Cu) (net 5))
 (segment (start 142.14 61.35) (end 141.5 61.99) (width 0.25) (layer B.Cu) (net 12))
 (segment (start 142.9 61.35) (end 142.14 61.35) (width 0.25) (layer B.Cu) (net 12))
 (segment (start 155.35 49.05) (end 155.3 49) (width 0.4) (layer B.Cu) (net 7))
 (segment (start 155.35 53.9) (end 155.35 52.92) (width 0.4) (layer B.Cu) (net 7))
 (segment (start 149.77 53.91) (end 149.77 52.28) (width 0.4) (layer B.Cu) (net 7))
 (segment (start 149.77 52.28) (end 151.18 50.87) (width 0.4) (layer B.Cu) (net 7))
 (segment (start 154.8 50.87) (end 155.35 51.42) (width 0.4) (layer B.Cu) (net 7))
 (segment (start 155.35 51.42) (end 155.35 49.05) (width 0.4) (layer B.Cu) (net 7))
 (segment (start 151.18 50.87) (end 154.8 50.87) (width 0.4) (layer B.Cu) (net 7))
 (segment (start 155.35 52.92) (end 155.35 51.42) (width 0.4) (layer B.Cu) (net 7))
 (segment (start 151.68 56.1) (end 151.67 56.11) (width 0.25) (layer B.Cu) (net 9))
 (segment (start 148.32 61.35) (end 147.02 61.35) (width 0.25) (layer B.Cu) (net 9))
 (segment (start 148.93 60.74) (end 148.32 61.35) (width 0.25) (layer B.Cu) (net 9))
 (segment (start 145.1 61.35) (end 147.02 61.35) (width 0.25) (layer B.Cu) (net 9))
 (segment (start 153.44 56.11) (end 153.45 56.1) (width 0.25) (layer B.Cu) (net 9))
 (segment (start 151.67 56.11) (end 153.44 56.11) (width 0.25) (layer B.Cu) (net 9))
 (segment (start 151.67 56.11) (end 151.67 56.91) (width 0.25) (layer B.Cu) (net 9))
 (segment (start 151.67 56.91) (end 151.35 57.23) (width 0.25) (layer B.Cu) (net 9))
 (segment (start 151.35 57.23) (end 149.86 57.23) (width 0.25) (layer B.Cu) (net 9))
 (segment (start 148.93 58.16) (end 148.93 60.74) (width 0.25) (layer B.Cu) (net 9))
 (segment (start 149.86 57.23) (end 148.93 58.16) (width 0.25) (layer B.Cu) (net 9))
 (segment (start 155.35 56.1) (end 155.35 58.28) (width 0.25) (layer B.Cu) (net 8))
 (segment (start 154.69 58.94) (end 153.51 58.94) (width 0.25) (layer B.Cu) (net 8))
 (via (at 153.51 58.94) (size 0.8) (drill 0.4) (layers F.Cu B.Cu) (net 8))
 (segment (start 155.35 58.28) (end 154.69 58.94) (width 0.25) (layer B.Cu) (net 8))
 (via (at 146.42 59.45) (size 0.8) (drill 0.4) (layers F.Cu B.Cu) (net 8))
 (segment (start 145.1 59.45) (end 146.42 59.45) (width 0.25) (layer B.Cu) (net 8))
 (segment (start 146.42 60.69) (end 146.42 59.45) (width 0.25) (layer F.Cu) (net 8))
 (segment (start 147.23 61.5) (end 146.42 60.69) (width 0.25) (layer F.Cu) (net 8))
 (segment (start 149.77 56.11) (end 148.92 56.11) (width 0.25) (layer B.Cu) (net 8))
 (segment (start 146.42 58.61) (end 146.42 59.45) (width 0.25) (layer B.Cu) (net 8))
 (segment (start 148.92 56.11) (end 146.42 58.61) (width 0.25) (layer B.Cu) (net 8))
 (segment (start 152.57 58.94) (end 150.01 61.5) (width 0.25) (layer F.Cu) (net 8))
 (segment (start 153.51 58.94) (end 152.57 58.94) (width 0.25) (layer F.Cu) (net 8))
 (segment (start 150.01 61.5) (end 147.23 61.5) (width 0.25) (layer F.Cu) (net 8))
 (segment (start 147.64 53.81) (end 147.64 56.42) (width 0.25) (layer B.Cu) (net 11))
 (segment (start 147.64 56.42) (end 146.29 57.77) (width 0.25) (layer B.Cu) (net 11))
 (segment (start 146.29 57.77) (end 143.66 57.77) (width 0.25) (layer B.Cu) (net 11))
 (segment (start 142.9 58.53) (end 142.9 59.45) (width 0.25) (layer B.Cu) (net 11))
 (segment (start 143.66 57.77) (end 142.9 58.53) (width 0.25) (layer B.Cu) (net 11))
 (segment (start 146.37 52.54) (end 147.64 53.81) (width 0.25) (layer B.Cu) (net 11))
 (segment (start 146.775 50.585) (end 146.37 50.99) (width 0.25) (layer B.Cu) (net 11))
 (segment (start 147.925 50.585) (end 146.775 50.585) (width 0.25) (layer B.Cu) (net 11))
 (segment (start 146.37 50.99) (end 146.37 52.54) (width 0.25) (layer B.Cu) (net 11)))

